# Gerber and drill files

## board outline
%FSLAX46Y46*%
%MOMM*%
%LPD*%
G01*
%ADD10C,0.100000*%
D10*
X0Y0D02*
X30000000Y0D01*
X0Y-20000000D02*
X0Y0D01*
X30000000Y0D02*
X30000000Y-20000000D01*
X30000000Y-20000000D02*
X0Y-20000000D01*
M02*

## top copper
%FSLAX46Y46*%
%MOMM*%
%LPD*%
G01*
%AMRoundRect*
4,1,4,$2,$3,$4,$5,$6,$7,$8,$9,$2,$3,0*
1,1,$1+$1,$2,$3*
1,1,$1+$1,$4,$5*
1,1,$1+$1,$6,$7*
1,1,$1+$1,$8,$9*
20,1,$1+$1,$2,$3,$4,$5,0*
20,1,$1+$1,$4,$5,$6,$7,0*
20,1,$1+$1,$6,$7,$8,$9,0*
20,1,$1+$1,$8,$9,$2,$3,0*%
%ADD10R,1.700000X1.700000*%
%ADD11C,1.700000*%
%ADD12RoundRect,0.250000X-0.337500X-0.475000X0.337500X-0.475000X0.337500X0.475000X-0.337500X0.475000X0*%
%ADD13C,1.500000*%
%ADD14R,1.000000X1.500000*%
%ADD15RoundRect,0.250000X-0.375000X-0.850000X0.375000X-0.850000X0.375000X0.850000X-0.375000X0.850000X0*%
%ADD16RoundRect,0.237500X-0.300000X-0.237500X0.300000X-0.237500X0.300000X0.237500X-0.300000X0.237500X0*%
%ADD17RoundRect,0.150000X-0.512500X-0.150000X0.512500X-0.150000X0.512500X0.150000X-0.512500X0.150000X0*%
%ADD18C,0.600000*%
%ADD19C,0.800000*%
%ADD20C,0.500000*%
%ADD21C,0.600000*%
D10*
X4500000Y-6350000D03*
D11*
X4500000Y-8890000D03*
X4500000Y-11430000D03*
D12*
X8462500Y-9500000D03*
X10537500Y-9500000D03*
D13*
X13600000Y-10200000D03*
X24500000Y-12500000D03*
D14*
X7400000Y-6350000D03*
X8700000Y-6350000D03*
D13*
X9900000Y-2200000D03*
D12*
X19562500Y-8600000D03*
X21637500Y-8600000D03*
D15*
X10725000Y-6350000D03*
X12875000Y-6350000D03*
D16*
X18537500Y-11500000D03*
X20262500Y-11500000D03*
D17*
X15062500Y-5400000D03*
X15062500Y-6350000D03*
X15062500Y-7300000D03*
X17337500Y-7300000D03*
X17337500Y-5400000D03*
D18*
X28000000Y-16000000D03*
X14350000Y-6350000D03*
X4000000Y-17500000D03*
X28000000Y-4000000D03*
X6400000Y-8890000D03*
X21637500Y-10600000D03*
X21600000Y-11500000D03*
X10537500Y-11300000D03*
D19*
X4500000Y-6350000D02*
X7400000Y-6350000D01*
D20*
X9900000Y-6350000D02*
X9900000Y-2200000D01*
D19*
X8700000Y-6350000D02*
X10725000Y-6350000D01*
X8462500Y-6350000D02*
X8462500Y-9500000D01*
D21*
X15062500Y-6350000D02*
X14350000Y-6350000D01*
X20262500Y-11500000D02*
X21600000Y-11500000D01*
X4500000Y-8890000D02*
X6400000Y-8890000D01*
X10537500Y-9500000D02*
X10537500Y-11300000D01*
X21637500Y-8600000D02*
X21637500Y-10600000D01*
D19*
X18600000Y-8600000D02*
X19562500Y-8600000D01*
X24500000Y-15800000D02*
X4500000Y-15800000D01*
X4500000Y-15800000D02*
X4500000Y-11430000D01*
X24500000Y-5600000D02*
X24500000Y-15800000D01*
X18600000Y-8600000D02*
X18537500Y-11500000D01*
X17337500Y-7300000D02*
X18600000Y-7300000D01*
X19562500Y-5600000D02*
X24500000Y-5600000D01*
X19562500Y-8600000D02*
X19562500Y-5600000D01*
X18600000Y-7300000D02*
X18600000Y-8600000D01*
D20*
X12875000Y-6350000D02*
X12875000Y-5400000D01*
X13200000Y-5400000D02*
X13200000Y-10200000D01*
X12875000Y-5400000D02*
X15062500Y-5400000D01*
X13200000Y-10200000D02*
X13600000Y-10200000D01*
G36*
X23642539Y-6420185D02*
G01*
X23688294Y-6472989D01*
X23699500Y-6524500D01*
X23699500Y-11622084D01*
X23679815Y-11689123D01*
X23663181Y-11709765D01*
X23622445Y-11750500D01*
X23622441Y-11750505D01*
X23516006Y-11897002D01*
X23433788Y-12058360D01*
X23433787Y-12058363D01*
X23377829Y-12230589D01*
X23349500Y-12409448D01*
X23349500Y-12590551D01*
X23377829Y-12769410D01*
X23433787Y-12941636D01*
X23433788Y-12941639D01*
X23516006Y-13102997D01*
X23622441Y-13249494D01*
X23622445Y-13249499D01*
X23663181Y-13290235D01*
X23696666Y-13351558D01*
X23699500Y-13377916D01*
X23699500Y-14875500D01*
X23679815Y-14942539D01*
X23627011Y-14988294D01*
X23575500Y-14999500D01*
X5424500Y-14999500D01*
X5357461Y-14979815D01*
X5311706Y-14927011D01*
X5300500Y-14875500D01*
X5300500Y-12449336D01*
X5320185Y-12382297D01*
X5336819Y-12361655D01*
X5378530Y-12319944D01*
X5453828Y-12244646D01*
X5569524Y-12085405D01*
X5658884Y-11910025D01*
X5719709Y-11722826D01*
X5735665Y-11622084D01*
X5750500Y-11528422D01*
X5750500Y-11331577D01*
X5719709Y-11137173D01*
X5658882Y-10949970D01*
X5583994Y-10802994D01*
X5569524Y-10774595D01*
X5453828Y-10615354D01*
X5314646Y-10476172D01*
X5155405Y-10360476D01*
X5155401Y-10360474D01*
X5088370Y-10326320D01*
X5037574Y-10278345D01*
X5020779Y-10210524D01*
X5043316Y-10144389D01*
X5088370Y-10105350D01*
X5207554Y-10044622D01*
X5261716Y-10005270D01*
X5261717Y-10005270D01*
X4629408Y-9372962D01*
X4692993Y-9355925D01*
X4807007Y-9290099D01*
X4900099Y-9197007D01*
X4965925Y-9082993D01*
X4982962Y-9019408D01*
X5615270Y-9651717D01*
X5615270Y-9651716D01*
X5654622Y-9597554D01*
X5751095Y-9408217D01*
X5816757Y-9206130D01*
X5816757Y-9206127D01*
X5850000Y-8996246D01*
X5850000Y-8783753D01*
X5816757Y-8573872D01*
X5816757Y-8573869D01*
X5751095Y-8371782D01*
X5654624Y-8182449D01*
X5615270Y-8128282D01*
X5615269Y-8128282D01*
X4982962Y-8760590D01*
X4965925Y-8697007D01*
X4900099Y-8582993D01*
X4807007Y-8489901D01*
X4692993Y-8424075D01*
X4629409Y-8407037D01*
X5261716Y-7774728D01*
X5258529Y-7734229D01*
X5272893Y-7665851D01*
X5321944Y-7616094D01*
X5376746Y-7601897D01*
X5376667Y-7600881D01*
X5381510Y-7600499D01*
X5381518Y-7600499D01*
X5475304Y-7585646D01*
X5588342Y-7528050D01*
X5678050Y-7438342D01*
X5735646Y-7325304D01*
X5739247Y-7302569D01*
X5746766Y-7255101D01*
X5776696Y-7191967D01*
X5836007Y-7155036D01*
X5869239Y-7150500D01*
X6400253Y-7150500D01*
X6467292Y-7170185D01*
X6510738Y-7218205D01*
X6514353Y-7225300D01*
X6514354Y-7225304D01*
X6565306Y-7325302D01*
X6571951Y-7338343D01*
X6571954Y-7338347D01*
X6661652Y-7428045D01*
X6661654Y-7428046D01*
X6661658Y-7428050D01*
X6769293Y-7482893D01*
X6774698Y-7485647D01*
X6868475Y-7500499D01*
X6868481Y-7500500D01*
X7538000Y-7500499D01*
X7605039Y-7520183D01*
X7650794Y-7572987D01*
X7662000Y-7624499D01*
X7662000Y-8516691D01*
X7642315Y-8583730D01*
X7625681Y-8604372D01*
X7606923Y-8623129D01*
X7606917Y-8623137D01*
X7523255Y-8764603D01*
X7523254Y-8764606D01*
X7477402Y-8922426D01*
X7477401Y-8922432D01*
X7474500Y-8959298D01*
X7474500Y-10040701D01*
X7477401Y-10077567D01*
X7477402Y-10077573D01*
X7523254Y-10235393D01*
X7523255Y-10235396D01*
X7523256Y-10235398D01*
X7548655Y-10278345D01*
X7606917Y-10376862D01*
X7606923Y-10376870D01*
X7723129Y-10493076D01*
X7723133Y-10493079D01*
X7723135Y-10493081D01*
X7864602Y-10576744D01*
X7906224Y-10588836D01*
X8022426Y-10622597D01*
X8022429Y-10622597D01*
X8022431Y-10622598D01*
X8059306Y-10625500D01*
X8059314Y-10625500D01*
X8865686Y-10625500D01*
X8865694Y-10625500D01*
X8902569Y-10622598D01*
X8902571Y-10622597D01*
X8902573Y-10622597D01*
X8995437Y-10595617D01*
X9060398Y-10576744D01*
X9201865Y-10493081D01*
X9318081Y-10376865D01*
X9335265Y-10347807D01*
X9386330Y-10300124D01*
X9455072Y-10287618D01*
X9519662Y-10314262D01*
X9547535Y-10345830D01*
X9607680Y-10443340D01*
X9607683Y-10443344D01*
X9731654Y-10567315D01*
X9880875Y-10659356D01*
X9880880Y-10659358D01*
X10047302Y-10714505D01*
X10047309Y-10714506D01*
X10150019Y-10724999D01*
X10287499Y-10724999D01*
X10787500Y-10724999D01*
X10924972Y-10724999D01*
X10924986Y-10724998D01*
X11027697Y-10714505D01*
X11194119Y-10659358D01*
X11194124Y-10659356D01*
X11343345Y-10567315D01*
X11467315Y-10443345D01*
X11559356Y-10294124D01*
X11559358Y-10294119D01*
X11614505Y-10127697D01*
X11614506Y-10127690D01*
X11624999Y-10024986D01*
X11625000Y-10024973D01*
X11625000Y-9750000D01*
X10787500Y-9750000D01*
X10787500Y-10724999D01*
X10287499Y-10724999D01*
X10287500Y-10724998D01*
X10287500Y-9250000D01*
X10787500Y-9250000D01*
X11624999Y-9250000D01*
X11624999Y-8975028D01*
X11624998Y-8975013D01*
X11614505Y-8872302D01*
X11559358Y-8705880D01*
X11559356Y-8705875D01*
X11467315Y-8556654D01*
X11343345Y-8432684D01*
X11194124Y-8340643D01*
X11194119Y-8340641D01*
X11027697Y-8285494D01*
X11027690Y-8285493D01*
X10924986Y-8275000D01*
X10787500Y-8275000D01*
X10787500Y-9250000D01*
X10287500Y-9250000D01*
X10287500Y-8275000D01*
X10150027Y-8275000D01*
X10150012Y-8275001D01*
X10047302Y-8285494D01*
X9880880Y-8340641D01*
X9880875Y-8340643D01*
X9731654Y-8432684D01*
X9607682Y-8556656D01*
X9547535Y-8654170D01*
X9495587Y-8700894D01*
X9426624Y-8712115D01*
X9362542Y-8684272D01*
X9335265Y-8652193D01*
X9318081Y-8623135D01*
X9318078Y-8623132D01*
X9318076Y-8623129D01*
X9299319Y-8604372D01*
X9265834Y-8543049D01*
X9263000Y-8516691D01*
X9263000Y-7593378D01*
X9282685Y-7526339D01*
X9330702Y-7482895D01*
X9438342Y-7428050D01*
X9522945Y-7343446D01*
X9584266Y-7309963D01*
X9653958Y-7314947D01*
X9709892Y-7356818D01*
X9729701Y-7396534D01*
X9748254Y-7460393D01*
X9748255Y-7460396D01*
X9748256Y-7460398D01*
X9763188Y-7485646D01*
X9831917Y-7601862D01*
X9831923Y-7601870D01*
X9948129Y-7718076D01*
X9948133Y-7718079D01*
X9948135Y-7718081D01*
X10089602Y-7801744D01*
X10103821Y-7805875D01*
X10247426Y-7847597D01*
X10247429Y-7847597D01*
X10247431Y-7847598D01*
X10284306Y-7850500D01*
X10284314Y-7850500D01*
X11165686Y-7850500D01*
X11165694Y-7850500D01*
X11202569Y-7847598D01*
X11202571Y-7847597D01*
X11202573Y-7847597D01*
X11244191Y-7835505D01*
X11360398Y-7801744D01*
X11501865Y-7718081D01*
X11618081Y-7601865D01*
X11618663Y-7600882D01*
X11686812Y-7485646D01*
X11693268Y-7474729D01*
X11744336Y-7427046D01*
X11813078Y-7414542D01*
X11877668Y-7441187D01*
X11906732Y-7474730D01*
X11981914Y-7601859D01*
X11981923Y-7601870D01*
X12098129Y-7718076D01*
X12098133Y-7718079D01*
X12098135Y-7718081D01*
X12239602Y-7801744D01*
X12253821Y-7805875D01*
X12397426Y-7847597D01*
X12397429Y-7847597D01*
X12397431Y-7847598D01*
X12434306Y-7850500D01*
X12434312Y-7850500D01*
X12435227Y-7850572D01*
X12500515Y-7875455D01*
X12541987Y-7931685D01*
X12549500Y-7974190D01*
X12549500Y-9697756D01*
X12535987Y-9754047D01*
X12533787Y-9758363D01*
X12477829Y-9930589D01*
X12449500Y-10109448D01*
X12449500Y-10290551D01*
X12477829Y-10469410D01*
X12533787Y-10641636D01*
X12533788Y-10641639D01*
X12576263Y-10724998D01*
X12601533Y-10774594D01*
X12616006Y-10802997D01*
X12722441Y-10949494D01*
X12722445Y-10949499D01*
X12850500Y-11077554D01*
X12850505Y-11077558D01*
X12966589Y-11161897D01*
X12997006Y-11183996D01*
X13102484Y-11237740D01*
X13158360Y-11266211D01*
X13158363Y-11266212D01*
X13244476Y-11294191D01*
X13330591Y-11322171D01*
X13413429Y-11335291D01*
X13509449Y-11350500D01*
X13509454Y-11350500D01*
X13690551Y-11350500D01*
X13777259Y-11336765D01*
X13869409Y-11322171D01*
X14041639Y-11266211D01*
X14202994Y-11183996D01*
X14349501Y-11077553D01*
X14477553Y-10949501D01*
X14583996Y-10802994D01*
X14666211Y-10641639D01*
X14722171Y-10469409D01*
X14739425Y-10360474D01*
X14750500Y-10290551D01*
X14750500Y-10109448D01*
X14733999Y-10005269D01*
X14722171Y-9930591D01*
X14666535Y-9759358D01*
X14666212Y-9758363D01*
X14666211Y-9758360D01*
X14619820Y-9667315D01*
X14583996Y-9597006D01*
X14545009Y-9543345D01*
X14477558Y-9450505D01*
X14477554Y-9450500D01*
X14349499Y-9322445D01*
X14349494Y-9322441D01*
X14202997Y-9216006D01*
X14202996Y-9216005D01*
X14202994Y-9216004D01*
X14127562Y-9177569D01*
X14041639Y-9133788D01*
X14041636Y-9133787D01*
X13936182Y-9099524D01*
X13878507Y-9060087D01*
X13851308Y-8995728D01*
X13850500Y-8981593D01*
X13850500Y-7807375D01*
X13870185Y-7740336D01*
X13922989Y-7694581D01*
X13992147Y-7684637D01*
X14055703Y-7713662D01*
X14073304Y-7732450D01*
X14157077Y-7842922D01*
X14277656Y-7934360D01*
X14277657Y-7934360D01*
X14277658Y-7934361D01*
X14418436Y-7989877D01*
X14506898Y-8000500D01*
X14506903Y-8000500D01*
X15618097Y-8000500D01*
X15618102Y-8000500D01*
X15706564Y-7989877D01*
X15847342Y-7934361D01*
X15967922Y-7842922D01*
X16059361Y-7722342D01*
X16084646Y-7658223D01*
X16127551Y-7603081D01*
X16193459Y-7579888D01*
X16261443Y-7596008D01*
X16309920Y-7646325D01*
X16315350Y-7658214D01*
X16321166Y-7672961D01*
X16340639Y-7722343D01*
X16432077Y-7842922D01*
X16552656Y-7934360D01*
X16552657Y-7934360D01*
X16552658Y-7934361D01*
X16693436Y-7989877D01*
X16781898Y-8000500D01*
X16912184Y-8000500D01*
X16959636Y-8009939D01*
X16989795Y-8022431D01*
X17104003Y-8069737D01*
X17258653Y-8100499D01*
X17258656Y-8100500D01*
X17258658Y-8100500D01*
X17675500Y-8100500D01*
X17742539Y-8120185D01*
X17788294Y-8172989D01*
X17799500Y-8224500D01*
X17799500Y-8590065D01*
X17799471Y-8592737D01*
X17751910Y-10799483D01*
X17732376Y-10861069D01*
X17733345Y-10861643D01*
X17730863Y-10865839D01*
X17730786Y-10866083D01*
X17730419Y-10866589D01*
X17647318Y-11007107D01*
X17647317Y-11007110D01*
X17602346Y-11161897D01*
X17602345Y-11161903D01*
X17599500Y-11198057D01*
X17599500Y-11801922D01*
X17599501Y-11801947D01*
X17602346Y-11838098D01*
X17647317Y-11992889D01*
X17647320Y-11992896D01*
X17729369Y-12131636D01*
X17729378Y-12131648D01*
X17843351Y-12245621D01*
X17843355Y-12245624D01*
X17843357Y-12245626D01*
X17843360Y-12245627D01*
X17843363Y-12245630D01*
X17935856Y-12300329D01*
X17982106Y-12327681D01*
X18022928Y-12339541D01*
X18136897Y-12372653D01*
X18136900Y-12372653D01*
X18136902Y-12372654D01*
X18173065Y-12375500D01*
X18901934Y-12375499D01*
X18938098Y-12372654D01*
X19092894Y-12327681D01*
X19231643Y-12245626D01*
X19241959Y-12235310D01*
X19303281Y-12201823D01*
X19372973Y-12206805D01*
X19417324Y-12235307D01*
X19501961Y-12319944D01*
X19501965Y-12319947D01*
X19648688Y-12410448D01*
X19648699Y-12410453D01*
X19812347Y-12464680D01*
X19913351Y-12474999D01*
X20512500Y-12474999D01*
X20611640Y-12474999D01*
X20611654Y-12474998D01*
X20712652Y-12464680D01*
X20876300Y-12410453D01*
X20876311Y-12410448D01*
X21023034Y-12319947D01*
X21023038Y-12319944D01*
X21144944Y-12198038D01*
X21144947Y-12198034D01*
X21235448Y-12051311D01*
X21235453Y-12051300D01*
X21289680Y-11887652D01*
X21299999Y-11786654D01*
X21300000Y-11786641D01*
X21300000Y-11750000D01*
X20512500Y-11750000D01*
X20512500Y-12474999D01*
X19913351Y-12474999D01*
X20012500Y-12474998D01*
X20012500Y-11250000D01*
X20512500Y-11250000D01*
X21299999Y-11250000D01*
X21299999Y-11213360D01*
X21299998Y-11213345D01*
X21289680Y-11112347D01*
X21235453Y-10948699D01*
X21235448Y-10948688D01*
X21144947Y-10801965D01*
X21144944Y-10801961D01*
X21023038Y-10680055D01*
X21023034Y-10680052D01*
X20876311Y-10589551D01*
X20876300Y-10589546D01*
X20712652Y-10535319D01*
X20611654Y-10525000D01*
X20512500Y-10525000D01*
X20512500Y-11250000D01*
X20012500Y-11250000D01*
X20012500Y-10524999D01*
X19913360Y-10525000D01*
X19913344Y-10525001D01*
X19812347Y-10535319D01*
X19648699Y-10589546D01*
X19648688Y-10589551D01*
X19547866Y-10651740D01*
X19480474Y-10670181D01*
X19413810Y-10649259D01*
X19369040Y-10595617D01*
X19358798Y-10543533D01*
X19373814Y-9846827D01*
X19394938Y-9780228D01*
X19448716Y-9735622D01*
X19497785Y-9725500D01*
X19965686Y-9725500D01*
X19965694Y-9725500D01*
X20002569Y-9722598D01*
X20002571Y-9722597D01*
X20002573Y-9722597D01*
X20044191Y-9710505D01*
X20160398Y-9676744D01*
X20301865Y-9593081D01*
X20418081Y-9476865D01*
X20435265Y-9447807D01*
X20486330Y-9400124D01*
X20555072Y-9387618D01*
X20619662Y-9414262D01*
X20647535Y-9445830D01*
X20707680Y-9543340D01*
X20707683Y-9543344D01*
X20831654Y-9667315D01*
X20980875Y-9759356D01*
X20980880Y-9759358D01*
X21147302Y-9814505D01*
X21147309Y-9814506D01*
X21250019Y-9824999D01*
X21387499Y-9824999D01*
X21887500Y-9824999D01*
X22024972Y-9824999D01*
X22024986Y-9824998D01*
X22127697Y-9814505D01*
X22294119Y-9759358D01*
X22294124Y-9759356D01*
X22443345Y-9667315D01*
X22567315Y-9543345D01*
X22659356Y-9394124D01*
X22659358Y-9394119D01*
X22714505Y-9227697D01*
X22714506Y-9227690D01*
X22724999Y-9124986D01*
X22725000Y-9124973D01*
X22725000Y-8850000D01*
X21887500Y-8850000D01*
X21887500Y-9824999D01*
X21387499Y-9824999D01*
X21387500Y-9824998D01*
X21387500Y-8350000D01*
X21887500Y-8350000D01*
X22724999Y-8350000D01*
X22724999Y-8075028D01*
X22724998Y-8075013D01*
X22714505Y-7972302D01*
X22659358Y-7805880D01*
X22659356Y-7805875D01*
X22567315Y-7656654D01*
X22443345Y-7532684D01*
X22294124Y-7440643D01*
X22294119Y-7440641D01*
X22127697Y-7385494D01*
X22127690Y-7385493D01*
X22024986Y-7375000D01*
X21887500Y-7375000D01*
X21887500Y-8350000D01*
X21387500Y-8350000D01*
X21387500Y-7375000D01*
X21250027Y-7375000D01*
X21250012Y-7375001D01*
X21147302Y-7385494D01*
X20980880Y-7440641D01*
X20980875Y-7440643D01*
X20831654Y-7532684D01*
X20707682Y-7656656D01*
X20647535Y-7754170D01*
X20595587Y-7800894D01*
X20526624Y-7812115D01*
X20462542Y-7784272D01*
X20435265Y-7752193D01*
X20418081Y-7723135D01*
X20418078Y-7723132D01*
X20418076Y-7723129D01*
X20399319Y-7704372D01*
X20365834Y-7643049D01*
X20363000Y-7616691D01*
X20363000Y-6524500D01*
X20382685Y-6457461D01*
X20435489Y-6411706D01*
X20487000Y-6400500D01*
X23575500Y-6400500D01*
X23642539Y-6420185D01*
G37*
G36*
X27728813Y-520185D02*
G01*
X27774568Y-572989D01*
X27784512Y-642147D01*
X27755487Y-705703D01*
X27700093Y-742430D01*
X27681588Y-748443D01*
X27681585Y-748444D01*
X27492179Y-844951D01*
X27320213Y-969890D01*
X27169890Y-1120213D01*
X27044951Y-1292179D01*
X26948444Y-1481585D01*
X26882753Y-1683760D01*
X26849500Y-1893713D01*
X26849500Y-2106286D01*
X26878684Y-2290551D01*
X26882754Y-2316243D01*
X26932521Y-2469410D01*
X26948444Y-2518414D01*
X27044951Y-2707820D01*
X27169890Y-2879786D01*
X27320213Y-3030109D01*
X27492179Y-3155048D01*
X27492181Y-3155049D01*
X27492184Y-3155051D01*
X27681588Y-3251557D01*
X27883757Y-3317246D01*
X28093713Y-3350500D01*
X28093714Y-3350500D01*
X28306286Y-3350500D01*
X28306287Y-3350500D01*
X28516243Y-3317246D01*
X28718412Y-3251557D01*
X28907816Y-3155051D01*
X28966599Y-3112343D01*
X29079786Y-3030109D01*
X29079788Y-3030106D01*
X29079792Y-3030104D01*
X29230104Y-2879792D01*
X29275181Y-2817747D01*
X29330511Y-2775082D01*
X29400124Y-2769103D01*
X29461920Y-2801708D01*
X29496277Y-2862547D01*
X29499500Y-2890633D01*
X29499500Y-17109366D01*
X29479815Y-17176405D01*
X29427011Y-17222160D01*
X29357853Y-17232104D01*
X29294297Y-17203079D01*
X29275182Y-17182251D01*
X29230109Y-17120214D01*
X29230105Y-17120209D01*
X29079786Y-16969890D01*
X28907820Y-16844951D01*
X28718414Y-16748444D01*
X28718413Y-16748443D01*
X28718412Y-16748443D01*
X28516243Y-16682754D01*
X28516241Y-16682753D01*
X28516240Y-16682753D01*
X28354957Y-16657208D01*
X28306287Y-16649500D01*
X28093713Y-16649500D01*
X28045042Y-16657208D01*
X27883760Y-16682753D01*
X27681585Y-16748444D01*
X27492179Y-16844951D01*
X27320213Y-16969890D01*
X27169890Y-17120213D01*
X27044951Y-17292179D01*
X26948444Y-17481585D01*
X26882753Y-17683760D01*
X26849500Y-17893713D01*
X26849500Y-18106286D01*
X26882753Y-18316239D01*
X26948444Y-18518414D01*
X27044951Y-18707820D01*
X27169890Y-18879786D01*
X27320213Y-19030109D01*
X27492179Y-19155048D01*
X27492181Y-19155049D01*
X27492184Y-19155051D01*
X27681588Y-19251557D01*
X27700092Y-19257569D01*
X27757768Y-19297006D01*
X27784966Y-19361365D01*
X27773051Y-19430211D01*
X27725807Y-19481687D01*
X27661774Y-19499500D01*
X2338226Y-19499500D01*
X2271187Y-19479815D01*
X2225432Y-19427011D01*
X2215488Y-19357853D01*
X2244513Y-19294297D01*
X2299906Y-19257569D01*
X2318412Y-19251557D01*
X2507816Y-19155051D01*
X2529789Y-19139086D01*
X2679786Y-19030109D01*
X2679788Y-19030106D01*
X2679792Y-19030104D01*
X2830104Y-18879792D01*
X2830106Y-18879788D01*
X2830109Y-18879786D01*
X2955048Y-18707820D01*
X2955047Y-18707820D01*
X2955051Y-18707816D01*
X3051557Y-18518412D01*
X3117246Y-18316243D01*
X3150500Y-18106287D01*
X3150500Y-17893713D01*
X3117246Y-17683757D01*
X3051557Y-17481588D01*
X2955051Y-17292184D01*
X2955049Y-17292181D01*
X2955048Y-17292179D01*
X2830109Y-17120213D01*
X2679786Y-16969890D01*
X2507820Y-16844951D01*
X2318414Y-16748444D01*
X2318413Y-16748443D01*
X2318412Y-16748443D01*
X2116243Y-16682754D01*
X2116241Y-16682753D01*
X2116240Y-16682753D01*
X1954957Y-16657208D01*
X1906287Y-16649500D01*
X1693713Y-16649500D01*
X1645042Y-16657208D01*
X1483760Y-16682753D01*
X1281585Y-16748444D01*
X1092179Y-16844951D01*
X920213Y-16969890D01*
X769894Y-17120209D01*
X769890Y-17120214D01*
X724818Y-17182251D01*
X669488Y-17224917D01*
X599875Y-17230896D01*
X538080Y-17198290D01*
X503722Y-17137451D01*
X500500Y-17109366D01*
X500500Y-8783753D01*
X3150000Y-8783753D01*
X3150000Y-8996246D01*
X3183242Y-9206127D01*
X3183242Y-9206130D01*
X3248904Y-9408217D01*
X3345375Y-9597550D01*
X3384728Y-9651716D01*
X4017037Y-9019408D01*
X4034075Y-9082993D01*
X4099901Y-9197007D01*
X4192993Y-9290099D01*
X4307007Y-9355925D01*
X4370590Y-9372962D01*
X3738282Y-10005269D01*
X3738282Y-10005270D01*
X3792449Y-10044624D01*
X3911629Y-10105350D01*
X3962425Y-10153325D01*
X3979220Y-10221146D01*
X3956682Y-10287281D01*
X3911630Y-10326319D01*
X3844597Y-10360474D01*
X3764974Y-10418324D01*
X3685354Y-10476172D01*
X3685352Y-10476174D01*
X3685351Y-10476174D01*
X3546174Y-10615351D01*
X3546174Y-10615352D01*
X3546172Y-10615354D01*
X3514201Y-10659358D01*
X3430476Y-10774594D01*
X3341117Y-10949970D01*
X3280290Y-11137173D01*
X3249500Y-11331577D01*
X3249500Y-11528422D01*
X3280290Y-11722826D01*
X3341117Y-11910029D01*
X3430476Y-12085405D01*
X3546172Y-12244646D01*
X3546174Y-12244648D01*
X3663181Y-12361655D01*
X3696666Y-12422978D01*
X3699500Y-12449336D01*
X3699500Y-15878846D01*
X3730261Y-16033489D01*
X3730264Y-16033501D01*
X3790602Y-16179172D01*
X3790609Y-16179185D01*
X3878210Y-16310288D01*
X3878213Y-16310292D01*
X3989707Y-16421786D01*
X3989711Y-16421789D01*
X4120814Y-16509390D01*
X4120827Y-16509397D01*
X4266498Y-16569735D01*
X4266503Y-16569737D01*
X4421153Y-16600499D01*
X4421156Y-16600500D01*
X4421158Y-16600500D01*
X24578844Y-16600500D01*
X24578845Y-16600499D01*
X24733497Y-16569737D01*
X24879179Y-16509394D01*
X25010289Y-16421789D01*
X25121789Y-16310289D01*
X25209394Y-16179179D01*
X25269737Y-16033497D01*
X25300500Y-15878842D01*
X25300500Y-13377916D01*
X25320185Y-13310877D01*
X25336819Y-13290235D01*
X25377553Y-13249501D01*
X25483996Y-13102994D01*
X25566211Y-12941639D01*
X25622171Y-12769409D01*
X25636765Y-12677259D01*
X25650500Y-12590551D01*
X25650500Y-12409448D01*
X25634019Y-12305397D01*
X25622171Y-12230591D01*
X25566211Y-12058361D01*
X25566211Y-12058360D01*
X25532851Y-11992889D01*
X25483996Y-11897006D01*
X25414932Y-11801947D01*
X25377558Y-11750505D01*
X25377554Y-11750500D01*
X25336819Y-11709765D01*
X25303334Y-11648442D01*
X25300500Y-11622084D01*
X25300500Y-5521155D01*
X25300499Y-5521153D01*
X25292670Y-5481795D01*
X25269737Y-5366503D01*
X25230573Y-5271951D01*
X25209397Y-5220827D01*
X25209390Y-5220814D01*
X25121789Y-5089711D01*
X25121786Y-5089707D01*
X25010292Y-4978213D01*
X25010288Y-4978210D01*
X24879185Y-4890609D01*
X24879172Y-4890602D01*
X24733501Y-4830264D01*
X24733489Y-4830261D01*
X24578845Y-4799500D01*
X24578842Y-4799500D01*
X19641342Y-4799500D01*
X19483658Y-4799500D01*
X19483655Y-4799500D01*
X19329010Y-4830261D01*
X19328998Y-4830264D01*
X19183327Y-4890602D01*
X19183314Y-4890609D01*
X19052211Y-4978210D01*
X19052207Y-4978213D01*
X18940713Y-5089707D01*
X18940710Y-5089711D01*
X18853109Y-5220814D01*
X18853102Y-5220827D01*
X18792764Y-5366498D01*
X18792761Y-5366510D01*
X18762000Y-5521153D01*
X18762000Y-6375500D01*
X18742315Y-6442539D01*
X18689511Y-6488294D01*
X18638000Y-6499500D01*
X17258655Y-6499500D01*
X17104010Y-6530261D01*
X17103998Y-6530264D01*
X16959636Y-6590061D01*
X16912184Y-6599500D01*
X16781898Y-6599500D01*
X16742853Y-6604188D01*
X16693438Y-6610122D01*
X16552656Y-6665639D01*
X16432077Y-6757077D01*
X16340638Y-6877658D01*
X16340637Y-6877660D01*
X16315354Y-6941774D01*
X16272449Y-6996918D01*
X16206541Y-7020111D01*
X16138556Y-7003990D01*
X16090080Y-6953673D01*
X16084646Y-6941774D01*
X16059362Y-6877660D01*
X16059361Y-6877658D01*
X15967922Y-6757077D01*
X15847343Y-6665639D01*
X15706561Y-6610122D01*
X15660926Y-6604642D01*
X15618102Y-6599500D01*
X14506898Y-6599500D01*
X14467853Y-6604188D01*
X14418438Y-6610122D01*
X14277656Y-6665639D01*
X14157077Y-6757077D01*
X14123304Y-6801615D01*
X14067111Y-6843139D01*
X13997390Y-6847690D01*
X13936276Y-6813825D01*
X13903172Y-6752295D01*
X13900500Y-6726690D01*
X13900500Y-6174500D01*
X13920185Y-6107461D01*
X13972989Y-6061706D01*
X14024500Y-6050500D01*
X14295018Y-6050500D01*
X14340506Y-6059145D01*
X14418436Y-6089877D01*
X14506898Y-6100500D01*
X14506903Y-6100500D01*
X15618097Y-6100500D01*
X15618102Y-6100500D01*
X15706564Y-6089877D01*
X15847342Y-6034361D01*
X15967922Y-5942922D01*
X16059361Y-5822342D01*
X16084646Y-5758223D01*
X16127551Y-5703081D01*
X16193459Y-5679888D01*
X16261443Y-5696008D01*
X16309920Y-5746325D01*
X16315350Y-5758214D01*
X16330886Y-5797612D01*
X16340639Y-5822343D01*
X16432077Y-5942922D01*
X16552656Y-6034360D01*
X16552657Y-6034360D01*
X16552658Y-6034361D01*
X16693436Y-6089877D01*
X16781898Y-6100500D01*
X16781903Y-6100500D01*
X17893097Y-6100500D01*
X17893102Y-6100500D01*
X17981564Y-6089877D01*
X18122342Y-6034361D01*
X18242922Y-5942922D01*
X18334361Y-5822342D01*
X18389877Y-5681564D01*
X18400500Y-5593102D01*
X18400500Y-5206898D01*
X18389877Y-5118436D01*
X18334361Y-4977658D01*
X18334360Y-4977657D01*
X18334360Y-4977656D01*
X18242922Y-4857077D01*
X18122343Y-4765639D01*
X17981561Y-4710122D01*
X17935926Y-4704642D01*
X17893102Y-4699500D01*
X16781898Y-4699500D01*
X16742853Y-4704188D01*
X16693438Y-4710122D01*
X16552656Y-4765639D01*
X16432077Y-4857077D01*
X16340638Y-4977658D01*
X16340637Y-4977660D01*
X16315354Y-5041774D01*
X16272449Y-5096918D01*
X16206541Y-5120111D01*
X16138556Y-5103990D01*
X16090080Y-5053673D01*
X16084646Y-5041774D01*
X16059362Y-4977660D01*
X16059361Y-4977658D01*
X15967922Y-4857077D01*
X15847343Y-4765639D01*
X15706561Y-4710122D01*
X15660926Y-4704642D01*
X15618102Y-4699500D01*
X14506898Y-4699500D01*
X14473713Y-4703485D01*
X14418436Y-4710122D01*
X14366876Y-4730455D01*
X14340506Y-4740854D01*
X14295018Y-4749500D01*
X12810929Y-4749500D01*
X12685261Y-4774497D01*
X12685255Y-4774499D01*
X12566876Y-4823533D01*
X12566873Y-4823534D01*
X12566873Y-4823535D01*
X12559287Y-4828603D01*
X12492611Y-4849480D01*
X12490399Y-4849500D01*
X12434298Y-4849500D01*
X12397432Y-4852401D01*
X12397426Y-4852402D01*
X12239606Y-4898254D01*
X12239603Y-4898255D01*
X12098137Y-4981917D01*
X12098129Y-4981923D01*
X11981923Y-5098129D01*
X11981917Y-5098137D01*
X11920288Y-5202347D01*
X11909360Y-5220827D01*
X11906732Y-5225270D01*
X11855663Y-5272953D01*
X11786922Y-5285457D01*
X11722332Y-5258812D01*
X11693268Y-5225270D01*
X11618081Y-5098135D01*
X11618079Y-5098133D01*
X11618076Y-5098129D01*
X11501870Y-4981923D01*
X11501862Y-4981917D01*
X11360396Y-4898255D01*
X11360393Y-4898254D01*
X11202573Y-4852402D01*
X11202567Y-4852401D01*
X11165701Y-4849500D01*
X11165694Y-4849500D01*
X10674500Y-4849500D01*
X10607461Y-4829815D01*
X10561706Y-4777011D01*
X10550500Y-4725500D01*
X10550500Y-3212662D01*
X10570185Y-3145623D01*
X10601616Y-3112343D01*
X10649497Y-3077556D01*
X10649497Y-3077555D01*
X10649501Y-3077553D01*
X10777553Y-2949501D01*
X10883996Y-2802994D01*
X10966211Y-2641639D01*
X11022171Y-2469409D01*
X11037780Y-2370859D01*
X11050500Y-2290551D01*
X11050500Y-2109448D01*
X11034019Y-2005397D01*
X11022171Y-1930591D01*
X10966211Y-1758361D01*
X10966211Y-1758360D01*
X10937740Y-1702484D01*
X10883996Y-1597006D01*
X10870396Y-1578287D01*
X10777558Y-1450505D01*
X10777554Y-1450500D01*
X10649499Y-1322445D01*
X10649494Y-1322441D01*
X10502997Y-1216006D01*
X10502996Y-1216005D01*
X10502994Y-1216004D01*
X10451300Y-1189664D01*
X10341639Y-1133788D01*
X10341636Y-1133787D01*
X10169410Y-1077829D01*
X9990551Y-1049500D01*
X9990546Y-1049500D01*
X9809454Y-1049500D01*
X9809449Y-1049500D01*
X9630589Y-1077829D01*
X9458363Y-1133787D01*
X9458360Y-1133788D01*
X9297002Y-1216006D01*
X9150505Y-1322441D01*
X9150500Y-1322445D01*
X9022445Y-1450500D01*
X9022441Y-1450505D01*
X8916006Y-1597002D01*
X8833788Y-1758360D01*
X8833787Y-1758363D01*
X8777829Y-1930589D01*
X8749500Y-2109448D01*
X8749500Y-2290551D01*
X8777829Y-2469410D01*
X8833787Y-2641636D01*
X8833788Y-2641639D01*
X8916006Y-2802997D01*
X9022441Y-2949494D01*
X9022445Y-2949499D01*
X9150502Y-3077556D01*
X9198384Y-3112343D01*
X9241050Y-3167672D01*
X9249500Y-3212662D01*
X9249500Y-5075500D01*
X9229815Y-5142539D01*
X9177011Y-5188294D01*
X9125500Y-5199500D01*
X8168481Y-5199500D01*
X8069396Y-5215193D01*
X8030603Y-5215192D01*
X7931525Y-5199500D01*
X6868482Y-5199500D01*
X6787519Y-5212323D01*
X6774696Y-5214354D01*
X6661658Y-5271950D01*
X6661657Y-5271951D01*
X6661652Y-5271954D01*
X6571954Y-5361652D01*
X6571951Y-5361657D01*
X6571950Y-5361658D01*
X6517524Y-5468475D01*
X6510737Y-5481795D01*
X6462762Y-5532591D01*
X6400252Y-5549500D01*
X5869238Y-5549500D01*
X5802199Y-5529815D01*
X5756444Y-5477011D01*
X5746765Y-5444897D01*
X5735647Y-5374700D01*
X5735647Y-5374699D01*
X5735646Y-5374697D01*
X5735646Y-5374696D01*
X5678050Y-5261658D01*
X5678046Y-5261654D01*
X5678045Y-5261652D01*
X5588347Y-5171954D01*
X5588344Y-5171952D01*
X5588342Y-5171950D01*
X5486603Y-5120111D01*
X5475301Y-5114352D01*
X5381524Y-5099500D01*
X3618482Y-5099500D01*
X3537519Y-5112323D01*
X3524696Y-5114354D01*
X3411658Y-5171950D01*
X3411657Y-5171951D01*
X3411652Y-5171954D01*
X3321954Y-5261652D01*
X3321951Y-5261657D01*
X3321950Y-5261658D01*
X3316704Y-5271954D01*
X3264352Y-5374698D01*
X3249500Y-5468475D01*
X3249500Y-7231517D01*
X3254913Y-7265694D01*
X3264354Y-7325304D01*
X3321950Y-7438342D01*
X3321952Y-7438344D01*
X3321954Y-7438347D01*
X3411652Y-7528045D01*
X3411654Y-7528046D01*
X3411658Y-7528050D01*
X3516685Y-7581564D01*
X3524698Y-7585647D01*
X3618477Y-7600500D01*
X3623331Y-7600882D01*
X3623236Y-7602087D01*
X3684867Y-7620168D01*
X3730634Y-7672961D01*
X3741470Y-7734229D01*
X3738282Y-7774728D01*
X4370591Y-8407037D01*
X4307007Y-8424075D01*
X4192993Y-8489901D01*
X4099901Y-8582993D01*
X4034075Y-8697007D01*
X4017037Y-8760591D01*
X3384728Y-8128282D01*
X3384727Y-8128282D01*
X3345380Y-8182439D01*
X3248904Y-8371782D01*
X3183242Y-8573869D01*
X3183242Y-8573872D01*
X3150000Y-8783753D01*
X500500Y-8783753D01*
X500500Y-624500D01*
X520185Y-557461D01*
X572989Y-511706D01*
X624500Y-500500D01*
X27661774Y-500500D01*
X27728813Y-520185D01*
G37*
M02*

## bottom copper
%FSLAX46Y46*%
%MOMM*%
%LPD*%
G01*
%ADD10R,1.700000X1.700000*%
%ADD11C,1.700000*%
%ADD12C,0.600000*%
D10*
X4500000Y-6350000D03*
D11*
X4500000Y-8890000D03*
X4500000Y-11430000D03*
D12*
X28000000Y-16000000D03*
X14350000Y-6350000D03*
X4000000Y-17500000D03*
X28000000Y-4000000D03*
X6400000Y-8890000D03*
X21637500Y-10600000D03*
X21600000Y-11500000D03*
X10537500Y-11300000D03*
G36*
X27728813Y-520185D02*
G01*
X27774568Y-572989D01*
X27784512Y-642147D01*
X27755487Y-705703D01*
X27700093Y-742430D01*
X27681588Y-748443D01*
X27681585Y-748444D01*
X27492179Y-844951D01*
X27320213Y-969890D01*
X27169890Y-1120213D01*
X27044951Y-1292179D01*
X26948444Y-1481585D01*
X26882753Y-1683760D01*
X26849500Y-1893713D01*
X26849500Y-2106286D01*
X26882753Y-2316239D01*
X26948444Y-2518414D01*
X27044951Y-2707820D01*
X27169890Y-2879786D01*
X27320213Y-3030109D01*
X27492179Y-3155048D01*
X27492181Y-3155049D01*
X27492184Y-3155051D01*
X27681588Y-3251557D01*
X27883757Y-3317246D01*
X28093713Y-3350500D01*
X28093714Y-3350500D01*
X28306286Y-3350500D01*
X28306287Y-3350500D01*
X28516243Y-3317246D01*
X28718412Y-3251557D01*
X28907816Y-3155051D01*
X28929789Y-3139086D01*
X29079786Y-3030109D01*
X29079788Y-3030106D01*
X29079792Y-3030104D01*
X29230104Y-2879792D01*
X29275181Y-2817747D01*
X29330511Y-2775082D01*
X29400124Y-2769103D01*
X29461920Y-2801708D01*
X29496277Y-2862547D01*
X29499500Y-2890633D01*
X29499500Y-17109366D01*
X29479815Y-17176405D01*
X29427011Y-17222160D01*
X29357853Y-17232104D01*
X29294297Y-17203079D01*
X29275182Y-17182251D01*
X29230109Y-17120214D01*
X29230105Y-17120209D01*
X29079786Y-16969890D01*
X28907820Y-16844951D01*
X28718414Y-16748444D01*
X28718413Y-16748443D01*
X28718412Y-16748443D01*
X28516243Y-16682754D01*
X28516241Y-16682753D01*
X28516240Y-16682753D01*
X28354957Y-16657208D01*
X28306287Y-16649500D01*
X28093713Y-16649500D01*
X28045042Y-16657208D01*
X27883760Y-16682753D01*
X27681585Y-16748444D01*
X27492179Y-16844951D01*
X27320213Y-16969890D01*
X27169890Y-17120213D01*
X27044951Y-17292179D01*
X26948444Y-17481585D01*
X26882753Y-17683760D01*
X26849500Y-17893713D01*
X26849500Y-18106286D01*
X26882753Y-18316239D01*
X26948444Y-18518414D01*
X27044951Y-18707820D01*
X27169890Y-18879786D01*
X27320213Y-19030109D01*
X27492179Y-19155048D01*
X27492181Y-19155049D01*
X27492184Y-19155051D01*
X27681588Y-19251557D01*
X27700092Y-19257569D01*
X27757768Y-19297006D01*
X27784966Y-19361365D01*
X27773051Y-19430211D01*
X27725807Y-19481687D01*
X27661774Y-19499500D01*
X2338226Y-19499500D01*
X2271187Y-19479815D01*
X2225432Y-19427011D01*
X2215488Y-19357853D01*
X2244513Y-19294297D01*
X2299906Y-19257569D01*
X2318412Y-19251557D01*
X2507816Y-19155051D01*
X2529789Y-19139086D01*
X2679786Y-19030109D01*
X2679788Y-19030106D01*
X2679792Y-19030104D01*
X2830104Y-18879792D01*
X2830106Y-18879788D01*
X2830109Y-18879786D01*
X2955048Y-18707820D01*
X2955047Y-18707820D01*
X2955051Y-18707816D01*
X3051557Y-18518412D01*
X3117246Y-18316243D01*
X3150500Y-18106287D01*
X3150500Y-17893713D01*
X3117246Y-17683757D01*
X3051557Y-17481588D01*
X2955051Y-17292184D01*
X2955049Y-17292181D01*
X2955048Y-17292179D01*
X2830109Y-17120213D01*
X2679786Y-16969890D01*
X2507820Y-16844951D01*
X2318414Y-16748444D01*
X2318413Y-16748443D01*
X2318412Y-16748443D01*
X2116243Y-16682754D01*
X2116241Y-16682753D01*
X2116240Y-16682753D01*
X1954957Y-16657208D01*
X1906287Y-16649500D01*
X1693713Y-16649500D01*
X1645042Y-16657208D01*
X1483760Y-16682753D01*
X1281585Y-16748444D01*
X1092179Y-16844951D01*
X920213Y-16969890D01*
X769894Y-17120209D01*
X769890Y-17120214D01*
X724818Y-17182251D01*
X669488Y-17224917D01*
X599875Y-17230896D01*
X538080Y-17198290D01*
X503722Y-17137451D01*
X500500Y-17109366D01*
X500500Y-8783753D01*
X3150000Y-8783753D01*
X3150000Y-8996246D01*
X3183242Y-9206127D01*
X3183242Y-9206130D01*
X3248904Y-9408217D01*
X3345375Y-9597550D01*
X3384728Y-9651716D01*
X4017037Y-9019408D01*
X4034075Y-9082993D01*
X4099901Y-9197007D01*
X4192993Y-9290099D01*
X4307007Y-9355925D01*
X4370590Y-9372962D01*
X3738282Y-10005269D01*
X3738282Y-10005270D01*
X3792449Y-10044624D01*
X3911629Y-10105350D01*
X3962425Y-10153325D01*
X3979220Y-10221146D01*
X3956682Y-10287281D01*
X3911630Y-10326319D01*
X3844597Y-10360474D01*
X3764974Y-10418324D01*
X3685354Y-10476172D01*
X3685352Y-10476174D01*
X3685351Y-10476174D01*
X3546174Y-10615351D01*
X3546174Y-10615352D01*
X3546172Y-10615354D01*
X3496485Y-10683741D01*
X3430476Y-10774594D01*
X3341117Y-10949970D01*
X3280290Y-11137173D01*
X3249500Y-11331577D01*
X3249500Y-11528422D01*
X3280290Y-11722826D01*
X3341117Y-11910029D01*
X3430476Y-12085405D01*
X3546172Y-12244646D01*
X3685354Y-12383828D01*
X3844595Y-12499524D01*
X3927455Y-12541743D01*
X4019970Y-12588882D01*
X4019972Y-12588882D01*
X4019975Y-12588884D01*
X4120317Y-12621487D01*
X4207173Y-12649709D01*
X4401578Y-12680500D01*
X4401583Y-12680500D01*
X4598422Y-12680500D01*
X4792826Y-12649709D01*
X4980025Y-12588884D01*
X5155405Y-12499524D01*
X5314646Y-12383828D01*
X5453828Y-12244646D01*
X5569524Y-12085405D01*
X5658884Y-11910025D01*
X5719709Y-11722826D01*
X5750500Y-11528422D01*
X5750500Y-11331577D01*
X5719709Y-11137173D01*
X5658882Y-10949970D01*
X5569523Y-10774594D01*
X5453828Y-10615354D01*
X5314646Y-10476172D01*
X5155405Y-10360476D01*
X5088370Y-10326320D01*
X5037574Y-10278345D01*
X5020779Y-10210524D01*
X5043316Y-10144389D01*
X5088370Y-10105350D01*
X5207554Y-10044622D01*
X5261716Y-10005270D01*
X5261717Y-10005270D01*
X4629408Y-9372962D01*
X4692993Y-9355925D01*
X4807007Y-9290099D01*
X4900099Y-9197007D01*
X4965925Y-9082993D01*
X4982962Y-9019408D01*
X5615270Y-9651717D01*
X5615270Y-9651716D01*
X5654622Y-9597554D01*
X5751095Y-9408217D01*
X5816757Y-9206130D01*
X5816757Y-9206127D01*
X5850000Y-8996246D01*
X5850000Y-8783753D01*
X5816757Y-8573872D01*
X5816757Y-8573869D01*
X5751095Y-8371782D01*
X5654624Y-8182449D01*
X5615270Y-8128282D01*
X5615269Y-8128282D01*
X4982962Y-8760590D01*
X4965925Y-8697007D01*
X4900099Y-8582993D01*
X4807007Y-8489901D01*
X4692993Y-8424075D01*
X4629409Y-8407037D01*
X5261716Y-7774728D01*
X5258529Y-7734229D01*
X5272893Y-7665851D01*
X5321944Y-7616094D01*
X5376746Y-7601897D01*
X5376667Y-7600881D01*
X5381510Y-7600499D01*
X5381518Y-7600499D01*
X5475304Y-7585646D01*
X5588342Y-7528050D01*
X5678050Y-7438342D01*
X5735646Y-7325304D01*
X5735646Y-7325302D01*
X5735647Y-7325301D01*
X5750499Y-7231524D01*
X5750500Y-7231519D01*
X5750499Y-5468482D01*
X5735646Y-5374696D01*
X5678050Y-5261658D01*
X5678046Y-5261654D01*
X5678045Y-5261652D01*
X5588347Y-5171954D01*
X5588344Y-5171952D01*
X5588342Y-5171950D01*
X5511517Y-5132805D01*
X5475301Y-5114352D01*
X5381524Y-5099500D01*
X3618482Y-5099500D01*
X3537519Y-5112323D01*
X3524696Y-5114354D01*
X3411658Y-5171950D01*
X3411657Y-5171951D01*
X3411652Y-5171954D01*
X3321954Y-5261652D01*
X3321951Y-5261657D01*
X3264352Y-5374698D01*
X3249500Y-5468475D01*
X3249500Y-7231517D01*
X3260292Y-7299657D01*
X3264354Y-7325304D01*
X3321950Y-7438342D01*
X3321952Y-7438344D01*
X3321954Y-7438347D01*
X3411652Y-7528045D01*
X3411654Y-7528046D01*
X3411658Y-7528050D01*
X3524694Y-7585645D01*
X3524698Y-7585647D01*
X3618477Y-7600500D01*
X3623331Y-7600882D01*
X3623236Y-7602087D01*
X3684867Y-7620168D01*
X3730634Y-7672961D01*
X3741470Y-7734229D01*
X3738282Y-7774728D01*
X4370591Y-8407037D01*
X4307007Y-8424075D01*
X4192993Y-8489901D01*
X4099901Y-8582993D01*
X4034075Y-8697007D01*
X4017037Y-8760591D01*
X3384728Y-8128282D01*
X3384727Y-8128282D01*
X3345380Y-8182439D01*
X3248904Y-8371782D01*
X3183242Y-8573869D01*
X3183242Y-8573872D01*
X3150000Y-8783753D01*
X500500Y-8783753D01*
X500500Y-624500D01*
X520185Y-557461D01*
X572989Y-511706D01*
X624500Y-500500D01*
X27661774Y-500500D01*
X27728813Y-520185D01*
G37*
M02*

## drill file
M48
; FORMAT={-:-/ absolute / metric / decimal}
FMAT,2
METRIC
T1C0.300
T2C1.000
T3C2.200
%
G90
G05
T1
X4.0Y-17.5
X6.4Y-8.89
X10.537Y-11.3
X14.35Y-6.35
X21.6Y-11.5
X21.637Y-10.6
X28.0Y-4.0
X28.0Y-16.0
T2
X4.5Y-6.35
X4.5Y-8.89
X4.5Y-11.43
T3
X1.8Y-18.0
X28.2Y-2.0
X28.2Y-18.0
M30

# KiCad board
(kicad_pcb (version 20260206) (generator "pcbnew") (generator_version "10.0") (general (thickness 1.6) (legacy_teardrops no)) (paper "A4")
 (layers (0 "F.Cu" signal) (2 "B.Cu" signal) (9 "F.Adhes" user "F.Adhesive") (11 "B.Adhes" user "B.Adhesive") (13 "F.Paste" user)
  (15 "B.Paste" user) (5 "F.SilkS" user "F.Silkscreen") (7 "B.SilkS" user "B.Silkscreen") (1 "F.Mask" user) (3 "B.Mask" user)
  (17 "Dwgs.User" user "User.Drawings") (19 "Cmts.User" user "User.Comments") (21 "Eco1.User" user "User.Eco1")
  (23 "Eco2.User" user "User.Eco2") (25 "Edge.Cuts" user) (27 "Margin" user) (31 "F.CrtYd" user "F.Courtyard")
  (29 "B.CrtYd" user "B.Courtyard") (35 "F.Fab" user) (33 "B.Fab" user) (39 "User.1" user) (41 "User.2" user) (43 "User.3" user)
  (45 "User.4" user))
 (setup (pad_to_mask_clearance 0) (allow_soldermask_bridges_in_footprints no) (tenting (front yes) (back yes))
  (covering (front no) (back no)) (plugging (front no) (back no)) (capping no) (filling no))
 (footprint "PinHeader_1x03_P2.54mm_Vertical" (layer "F.Cu") (at 4.5 6.35)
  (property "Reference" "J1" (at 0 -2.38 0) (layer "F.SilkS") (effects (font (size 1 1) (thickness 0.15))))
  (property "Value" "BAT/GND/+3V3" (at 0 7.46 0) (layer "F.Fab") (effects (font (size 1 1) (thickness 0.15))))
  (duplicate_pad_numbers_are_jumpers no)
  (pad "1" thru_hole rect (at 0 0) (size 1.7 1.7) (drill 1) (layers "*.Cu" "*.Mask") (remove_unused_layers no) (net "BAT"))
  (pad "2" thru_hole circle (at 0 2.54) (size 1.7 1.7) (drill 1) (layers "*.Cu" "*.Mask") (remove_unused_layers no) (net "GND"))
  (pad "3" thru_hole circle (at 0 5.08) (size 1.7 1.7) (drill 1) (layers "*.Cu" "*.Mask") (remove_unused_layers no) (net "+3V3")))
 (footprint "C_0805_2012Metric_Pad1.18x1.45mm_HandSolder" (layer "F.Cu") (at 9.5 9.5)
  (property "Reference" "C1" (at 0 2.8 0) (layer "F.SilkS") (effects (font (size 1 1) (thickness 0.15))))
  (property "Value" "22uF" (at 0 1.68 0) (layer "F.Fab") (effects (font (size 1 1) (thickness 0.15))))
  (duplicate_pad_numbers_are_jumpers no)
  (pad "1" smd roundrect (at -1.0375 0) (size 1.175 1.45) (layers "F.Cu" "F.Mask" "F.Paste") (roundrect_rratio 0.212766) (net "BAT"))
  (pad "2" smd roundrect (at 1.0375 0) (size 1.175 1.45) (layers "F.Cu" "F.Mask" "F.Paste") (roundrect_rratio 0.212766) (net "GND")))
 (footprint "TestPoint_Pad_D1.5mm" (layer "F.Cu") (at 13.6 10.2)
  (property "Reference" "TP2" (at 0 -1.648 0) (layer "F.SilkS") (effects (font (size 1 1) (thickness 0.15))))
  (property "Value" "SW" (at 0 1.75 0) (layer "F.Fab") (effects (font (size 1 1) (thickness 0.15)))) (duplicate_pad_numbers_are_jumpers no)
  (pad "1" smd circle (at 0 0) (size 1.5 1.5) (layers "F.Cu" "F.Mask") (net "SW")))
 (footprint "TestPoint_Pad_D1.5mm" (layer "F.Cu") (at 24.5 12.5)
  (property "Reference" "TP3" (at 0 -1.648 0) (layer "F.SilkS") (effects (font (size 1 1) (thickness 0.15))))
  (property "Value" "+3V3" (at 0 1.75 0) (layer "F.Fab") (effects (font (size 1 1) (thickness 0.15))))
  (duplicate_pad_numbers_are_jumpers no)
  (pad "1" smd circle (at 0 0) (size 1.5 1.5) (layers "F.Cu" "F.Mask") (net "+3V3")))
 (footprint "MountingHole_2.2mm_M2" (layer "F.Cu") (at 1.8 18)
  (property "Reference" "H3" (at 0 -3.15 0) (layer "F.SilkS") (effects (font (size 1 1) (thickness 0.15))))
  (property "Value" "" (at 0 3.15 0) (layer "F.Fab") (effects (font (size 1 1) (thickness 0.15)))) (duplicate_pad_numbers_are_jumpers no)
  (pad "" np_thru_hole circle (at 0 0) (size 2.2 2.2) (drill 2.2) (layers "*.Cu" "*.Mask")))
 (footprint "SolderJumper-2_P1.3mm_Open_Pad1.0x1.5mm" (layer "F.Cu") (at 8.05 6.35)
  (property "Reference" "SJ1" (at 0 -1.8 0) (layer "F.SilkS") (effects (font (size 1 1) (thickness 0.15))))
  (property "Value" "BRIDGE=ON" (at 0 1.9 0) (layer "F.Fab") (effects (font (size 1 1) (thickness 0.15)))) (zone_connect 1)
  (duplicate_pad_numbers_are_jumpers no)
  (pad "1" smd rect (at -0.65 0) (size 1 1.5) (layers "F.Cu" "F.Mask") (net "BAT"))
  (pad "2" smd rect (at 0.65 0) (size 1 1.5) (layers "F.Cu" "F.Mask") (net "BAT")))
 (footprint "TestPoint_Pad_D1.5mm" (layer "F.Cu") (at 9.9 2.2)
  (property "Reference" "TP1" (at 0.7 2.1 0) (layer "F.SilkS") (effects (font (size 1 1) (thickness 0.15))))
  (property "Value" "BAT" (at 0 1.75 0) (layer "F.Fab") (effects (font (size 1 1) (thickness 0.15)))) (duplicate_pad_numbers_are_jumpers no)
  (pad "1" smd circle (at 0 0) (size 1.5 1.5) (layers "F.Cu" "F.Mask") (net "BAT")))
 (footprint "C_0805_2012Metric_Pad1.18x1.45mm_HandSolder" (layer "F.Cu") (at 20.6 8.6)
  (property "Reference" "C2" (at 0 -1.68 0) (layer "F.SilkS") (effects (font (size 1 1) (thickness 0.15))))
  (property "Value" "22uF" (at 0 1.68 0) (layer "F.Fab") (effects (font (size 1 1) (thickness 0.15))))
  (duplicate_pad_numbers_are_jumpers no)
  (pad "1" smd roundrect (at -1.0375 0) (size 1.175 1.45) (layers "F.Cu" "F.Mask" "F.Paste") (roundrect_rratio 0.212766) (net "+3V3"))
  (pad "2" smd roundrect (at 1.0375 0) (size 1.175 1.45) (layers "F.Cu" "F.Mask" "F.Paste") (roundrect_rratio 0.212766) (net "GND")))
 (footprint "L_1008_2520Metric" (layer "F.Cu") (at 11.8 6.35)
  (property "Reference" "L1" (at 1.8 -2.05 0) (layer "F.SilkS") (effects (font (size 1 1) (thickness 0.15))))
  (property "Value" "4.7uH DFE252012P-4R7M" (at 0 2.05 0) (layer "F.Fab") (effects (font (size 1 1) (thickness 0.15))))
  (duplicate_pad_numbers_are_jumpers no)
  (pad "1" smd roundrect (at -1.075 0) (size 1.25 2.2) (layers "F.Cu" "F.Mask" "F.Paste") (roundrect_rratio 0.2) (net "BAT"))
  (pad "2" smd roundrect (at 1.075 0) (size 1.25 2.2) (layers "F.Cu" "F.Mask" "F.Paste") (roundrect_rratio 0.2) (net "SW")))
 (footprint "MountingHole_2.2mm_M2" (layer "F.Cu") (at 28.2 18)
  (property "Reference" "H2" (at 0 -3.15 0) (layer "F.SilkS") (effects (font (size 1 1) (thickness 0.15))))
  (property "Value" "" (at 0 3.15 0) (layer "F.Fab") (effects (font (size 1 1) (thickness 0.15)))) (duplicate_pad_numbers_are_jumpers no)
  (pad "" np_thru_hole circle (at 0 0) (size 2.2 2.2) (drill 2.2) (layers "*.Cu" "*.Mask")))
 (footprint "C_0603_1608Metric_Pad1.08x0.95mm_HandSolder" (layer "F.Cu") (at 19.4 11.5)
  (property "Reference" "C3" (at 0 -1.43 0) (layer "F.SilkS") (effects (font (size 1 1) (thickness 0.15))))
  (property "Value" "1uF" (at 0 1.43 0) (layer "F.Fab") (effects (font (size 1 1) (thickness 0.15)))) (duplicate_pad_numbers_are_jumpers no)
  (pad "1" smd roundrect (at -0.8625 0) (size 1.075 0.95) (layers "F.Cu" "F.Mask" "F.Paste") (roundrect_rratio 0.25) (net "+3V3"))
  (pad "2" smd roundrect (at 0.8625 0) (size 1.075 0.95) (layers "F.Cu" "F.Mask" "F.Paste") (roundrect_rratio 0.25) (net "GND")))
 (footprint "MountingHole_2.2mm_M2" (layer "F.Cu") (at 28.2 2)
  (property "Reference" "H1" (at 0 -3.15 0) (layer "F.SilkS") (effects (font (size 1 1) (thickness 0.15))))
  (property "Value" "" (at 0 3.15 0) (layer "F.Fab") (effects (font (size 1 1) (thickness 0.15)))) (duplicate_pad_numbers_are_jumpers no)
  (pad "" np_thru_hole circle (at 0 0) (size 2.2 2.2) (drill 2.2) (layers "*.Cu" "*.Mask")))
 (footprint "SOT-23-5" (layer "F.Cu") (at 16.2 6.35)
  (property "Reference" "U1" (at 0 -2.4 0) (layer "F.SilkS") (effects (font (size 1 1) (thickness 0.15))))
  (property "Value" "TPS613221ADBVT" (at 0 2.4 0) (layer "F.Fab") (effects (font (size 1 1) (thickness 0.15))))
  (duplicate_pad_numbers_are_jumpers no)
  (pad "1" smd roundrect (at -1.1375 -0.95) (size 1.325 0.6) (layers "F.Cu" "F.Mask" "F.Paste") (roundrect_rratio 0.25) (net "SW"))
  (pad "2" smd roundrect (at -1.1375 0) (size 1.325 0.6) (layers "F.Cu" "F.Mask" "F.Paste") (roundrect_rratio 0.25) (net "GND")
   (zone_connect 2))
  (pad "3" smd roundrect (at -1.1375 0.95) (size 1.325 0.6) (layers "F.Cu" "F.Mask" "F.Paste") (roundrect_rratio 0.25))
  (pad "4" smd roundrect (at 1.1375 0.95) (size 1.325 0.6) (layers "F.Cu" "F.Mask" "F.Paste") (roundrect_rratio 0.25) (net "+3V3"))
  (pad "5" smd roundrect (at 1.1375 -0.95) (size 1.325 0.6) (layers "F.Cu" "F.Mask" "F.Paste") (roundrect_rratio 0.25)))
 (gr_line (start 0 0) (end 30 0) (stroke (width 0.1) (type default)) (layer "Edge.Cuts"))
 (gr_line (start 0 20) (end 0 0) (stroke (width 0.1) (type default)) (layer "Edge.Cuts"))
 (gr_line (start 30 0) (end 30 20) (stroke (width 0.1) (type default)) (layer "Edge.Cuts"))
 (gr_line (start 30 20) (end 0 20) (stroke (width 0.1) (type default)) (layer "Edge.Cuts"))
 (segment (start 4.5 6.35) (end 7.4 6.35) (width 0.8) (layer "F.Cu") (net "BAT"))
 (segment (start 9.9 6.35) (end 9.9 2.2) (width 0.5) (layer "F.Cu") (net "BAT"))
 (segment (start 8.7 6.35) (end 10.725 6.35) (width 0.8) (layer "F.Cu") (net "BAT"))
 (segment (start 8.4625 6.35) (end 8.4625 9.5) (width 0.8) (layer "F.Cu") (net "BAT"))
 (segment (start 15.0625 6.35) (end 14.35 6.35) (width 0.6) (layer "F.Cu") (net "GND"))
 (segment (start 20.2625 11.5) (end 21.6 11.5) (width 0.6) (layer "F.Cu") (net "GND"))
 (segment (start 4.5 8.89) (end 6.4 8.89) (width 0.6) (layer "F.Cu") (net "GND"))
 (segment (start 10.5375 9.5) (end 10.5375 11.3) (width 0.6) (layer "F.Cu") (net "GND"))
 (segment (start 21.6375 8.6) (end 21.6375 10.6) (width 0.6) (layer "F.Cu") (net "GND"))
 (via (at 28 16) (size 0.6) (drill 0.3) (layers "F.Cu" "B.Cu") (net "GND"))
 (via (at 14.35 6.35) (size 0.6) (drill 0.3) (layers "F.Cu" "B.Cu") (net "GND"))
 (via (at 4 17.5) (size 0.6) (drill 0.3) (layers "F.Cu" "B.Cu") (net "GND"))
 (via (at 28 4) (size 0.6) (drill 0.3) (layers "F.Cu" "B.Cu") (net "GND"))
 (via (at 6.4 8.89) (size 0.6) (drill 0.3) (layers "F.Cu" "B.Cu") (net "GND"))
 (via (at 21.6375 10.6) (size 0.6) (drill 0.3) (layers "F.Cu" "B.Cu") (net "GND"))
 (via (at 21.6 11.5) (size 0.6) (drill 0.3) (layers "F.Cu" "B.Cu") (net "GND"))
 (via (at 10.5375 11.3) (size 0.6) (drill 0.3) (layers "F.Cu" "B.Cu") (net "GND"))
 (segment (start 18.6 8.6) (end 19.5625 8.6) (width 0.8) (layer "F.Cu") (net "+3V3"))
 (segment (start 24.5 15.8) (end 4.5 15.8) (width 0.8) (layer "F.Cu") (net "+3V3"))
 (segment (start 4.5 15.8) (end 4.5 11.43) (width 0.8) (layer "F.Cu") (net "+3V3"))
 (segment (start 24.5 5.6) (end 24.5 15.8) (width 0.8) (layer "F.Cu") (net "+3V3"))
 (segment (start 18.6 8.6) (end 18.5375 11.5) (width 0.8) (layer "F.Cu") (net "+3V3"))
 (segment (start 17.3375 7.3) (end 18.6 7.3) (width 0.8) (layer "F.Cu") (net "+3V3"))
 (segment (start 19.5625 5.6) (end 24.5 5.6) (width 0.8) (layer "F.Cu") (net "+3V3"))
 (segment (start 19.5625 8.6) (end 19.5625 5.6) (width 0.8) (layer "F.Cu") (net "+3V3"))
 (segment (start 18.6 7.3) (end 18.6 8.6) (width 0.8) (layer "F.Cu") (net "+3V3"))
 (segment (start 12.875 6.35) (end 12.875 5.4) (width 0.5) (layer "F.Cu") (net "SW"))
 (segment (start 13.2 5.4) (end 13.2 10.2) (width 0.5) (layer "F.Cu") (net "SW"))
 (segment (start 12.875 5.4) (end 15.0625 5.4) (width 0.5) (layer "F.Cu") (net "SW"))
 (segment (start 13.2 10.2) (end 13.6 10.2) (width 0.5) (layer "F.Cu") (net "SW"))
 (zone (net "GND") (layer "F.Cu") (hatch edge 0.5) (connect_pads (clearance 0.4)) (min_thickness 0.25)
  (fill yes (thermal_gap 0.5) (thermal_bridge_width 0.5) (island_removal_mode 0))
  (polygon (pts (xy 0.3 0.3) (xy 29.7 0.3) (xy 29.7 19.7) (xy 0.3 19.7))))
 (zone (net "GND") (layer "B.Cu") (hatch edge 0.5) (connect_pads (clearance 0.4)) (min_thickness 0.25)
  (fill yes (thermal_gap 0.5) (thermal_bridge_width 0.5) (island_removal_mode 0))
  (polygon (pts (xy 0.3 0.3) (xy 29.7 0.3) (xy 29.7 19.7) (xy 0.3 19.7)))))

